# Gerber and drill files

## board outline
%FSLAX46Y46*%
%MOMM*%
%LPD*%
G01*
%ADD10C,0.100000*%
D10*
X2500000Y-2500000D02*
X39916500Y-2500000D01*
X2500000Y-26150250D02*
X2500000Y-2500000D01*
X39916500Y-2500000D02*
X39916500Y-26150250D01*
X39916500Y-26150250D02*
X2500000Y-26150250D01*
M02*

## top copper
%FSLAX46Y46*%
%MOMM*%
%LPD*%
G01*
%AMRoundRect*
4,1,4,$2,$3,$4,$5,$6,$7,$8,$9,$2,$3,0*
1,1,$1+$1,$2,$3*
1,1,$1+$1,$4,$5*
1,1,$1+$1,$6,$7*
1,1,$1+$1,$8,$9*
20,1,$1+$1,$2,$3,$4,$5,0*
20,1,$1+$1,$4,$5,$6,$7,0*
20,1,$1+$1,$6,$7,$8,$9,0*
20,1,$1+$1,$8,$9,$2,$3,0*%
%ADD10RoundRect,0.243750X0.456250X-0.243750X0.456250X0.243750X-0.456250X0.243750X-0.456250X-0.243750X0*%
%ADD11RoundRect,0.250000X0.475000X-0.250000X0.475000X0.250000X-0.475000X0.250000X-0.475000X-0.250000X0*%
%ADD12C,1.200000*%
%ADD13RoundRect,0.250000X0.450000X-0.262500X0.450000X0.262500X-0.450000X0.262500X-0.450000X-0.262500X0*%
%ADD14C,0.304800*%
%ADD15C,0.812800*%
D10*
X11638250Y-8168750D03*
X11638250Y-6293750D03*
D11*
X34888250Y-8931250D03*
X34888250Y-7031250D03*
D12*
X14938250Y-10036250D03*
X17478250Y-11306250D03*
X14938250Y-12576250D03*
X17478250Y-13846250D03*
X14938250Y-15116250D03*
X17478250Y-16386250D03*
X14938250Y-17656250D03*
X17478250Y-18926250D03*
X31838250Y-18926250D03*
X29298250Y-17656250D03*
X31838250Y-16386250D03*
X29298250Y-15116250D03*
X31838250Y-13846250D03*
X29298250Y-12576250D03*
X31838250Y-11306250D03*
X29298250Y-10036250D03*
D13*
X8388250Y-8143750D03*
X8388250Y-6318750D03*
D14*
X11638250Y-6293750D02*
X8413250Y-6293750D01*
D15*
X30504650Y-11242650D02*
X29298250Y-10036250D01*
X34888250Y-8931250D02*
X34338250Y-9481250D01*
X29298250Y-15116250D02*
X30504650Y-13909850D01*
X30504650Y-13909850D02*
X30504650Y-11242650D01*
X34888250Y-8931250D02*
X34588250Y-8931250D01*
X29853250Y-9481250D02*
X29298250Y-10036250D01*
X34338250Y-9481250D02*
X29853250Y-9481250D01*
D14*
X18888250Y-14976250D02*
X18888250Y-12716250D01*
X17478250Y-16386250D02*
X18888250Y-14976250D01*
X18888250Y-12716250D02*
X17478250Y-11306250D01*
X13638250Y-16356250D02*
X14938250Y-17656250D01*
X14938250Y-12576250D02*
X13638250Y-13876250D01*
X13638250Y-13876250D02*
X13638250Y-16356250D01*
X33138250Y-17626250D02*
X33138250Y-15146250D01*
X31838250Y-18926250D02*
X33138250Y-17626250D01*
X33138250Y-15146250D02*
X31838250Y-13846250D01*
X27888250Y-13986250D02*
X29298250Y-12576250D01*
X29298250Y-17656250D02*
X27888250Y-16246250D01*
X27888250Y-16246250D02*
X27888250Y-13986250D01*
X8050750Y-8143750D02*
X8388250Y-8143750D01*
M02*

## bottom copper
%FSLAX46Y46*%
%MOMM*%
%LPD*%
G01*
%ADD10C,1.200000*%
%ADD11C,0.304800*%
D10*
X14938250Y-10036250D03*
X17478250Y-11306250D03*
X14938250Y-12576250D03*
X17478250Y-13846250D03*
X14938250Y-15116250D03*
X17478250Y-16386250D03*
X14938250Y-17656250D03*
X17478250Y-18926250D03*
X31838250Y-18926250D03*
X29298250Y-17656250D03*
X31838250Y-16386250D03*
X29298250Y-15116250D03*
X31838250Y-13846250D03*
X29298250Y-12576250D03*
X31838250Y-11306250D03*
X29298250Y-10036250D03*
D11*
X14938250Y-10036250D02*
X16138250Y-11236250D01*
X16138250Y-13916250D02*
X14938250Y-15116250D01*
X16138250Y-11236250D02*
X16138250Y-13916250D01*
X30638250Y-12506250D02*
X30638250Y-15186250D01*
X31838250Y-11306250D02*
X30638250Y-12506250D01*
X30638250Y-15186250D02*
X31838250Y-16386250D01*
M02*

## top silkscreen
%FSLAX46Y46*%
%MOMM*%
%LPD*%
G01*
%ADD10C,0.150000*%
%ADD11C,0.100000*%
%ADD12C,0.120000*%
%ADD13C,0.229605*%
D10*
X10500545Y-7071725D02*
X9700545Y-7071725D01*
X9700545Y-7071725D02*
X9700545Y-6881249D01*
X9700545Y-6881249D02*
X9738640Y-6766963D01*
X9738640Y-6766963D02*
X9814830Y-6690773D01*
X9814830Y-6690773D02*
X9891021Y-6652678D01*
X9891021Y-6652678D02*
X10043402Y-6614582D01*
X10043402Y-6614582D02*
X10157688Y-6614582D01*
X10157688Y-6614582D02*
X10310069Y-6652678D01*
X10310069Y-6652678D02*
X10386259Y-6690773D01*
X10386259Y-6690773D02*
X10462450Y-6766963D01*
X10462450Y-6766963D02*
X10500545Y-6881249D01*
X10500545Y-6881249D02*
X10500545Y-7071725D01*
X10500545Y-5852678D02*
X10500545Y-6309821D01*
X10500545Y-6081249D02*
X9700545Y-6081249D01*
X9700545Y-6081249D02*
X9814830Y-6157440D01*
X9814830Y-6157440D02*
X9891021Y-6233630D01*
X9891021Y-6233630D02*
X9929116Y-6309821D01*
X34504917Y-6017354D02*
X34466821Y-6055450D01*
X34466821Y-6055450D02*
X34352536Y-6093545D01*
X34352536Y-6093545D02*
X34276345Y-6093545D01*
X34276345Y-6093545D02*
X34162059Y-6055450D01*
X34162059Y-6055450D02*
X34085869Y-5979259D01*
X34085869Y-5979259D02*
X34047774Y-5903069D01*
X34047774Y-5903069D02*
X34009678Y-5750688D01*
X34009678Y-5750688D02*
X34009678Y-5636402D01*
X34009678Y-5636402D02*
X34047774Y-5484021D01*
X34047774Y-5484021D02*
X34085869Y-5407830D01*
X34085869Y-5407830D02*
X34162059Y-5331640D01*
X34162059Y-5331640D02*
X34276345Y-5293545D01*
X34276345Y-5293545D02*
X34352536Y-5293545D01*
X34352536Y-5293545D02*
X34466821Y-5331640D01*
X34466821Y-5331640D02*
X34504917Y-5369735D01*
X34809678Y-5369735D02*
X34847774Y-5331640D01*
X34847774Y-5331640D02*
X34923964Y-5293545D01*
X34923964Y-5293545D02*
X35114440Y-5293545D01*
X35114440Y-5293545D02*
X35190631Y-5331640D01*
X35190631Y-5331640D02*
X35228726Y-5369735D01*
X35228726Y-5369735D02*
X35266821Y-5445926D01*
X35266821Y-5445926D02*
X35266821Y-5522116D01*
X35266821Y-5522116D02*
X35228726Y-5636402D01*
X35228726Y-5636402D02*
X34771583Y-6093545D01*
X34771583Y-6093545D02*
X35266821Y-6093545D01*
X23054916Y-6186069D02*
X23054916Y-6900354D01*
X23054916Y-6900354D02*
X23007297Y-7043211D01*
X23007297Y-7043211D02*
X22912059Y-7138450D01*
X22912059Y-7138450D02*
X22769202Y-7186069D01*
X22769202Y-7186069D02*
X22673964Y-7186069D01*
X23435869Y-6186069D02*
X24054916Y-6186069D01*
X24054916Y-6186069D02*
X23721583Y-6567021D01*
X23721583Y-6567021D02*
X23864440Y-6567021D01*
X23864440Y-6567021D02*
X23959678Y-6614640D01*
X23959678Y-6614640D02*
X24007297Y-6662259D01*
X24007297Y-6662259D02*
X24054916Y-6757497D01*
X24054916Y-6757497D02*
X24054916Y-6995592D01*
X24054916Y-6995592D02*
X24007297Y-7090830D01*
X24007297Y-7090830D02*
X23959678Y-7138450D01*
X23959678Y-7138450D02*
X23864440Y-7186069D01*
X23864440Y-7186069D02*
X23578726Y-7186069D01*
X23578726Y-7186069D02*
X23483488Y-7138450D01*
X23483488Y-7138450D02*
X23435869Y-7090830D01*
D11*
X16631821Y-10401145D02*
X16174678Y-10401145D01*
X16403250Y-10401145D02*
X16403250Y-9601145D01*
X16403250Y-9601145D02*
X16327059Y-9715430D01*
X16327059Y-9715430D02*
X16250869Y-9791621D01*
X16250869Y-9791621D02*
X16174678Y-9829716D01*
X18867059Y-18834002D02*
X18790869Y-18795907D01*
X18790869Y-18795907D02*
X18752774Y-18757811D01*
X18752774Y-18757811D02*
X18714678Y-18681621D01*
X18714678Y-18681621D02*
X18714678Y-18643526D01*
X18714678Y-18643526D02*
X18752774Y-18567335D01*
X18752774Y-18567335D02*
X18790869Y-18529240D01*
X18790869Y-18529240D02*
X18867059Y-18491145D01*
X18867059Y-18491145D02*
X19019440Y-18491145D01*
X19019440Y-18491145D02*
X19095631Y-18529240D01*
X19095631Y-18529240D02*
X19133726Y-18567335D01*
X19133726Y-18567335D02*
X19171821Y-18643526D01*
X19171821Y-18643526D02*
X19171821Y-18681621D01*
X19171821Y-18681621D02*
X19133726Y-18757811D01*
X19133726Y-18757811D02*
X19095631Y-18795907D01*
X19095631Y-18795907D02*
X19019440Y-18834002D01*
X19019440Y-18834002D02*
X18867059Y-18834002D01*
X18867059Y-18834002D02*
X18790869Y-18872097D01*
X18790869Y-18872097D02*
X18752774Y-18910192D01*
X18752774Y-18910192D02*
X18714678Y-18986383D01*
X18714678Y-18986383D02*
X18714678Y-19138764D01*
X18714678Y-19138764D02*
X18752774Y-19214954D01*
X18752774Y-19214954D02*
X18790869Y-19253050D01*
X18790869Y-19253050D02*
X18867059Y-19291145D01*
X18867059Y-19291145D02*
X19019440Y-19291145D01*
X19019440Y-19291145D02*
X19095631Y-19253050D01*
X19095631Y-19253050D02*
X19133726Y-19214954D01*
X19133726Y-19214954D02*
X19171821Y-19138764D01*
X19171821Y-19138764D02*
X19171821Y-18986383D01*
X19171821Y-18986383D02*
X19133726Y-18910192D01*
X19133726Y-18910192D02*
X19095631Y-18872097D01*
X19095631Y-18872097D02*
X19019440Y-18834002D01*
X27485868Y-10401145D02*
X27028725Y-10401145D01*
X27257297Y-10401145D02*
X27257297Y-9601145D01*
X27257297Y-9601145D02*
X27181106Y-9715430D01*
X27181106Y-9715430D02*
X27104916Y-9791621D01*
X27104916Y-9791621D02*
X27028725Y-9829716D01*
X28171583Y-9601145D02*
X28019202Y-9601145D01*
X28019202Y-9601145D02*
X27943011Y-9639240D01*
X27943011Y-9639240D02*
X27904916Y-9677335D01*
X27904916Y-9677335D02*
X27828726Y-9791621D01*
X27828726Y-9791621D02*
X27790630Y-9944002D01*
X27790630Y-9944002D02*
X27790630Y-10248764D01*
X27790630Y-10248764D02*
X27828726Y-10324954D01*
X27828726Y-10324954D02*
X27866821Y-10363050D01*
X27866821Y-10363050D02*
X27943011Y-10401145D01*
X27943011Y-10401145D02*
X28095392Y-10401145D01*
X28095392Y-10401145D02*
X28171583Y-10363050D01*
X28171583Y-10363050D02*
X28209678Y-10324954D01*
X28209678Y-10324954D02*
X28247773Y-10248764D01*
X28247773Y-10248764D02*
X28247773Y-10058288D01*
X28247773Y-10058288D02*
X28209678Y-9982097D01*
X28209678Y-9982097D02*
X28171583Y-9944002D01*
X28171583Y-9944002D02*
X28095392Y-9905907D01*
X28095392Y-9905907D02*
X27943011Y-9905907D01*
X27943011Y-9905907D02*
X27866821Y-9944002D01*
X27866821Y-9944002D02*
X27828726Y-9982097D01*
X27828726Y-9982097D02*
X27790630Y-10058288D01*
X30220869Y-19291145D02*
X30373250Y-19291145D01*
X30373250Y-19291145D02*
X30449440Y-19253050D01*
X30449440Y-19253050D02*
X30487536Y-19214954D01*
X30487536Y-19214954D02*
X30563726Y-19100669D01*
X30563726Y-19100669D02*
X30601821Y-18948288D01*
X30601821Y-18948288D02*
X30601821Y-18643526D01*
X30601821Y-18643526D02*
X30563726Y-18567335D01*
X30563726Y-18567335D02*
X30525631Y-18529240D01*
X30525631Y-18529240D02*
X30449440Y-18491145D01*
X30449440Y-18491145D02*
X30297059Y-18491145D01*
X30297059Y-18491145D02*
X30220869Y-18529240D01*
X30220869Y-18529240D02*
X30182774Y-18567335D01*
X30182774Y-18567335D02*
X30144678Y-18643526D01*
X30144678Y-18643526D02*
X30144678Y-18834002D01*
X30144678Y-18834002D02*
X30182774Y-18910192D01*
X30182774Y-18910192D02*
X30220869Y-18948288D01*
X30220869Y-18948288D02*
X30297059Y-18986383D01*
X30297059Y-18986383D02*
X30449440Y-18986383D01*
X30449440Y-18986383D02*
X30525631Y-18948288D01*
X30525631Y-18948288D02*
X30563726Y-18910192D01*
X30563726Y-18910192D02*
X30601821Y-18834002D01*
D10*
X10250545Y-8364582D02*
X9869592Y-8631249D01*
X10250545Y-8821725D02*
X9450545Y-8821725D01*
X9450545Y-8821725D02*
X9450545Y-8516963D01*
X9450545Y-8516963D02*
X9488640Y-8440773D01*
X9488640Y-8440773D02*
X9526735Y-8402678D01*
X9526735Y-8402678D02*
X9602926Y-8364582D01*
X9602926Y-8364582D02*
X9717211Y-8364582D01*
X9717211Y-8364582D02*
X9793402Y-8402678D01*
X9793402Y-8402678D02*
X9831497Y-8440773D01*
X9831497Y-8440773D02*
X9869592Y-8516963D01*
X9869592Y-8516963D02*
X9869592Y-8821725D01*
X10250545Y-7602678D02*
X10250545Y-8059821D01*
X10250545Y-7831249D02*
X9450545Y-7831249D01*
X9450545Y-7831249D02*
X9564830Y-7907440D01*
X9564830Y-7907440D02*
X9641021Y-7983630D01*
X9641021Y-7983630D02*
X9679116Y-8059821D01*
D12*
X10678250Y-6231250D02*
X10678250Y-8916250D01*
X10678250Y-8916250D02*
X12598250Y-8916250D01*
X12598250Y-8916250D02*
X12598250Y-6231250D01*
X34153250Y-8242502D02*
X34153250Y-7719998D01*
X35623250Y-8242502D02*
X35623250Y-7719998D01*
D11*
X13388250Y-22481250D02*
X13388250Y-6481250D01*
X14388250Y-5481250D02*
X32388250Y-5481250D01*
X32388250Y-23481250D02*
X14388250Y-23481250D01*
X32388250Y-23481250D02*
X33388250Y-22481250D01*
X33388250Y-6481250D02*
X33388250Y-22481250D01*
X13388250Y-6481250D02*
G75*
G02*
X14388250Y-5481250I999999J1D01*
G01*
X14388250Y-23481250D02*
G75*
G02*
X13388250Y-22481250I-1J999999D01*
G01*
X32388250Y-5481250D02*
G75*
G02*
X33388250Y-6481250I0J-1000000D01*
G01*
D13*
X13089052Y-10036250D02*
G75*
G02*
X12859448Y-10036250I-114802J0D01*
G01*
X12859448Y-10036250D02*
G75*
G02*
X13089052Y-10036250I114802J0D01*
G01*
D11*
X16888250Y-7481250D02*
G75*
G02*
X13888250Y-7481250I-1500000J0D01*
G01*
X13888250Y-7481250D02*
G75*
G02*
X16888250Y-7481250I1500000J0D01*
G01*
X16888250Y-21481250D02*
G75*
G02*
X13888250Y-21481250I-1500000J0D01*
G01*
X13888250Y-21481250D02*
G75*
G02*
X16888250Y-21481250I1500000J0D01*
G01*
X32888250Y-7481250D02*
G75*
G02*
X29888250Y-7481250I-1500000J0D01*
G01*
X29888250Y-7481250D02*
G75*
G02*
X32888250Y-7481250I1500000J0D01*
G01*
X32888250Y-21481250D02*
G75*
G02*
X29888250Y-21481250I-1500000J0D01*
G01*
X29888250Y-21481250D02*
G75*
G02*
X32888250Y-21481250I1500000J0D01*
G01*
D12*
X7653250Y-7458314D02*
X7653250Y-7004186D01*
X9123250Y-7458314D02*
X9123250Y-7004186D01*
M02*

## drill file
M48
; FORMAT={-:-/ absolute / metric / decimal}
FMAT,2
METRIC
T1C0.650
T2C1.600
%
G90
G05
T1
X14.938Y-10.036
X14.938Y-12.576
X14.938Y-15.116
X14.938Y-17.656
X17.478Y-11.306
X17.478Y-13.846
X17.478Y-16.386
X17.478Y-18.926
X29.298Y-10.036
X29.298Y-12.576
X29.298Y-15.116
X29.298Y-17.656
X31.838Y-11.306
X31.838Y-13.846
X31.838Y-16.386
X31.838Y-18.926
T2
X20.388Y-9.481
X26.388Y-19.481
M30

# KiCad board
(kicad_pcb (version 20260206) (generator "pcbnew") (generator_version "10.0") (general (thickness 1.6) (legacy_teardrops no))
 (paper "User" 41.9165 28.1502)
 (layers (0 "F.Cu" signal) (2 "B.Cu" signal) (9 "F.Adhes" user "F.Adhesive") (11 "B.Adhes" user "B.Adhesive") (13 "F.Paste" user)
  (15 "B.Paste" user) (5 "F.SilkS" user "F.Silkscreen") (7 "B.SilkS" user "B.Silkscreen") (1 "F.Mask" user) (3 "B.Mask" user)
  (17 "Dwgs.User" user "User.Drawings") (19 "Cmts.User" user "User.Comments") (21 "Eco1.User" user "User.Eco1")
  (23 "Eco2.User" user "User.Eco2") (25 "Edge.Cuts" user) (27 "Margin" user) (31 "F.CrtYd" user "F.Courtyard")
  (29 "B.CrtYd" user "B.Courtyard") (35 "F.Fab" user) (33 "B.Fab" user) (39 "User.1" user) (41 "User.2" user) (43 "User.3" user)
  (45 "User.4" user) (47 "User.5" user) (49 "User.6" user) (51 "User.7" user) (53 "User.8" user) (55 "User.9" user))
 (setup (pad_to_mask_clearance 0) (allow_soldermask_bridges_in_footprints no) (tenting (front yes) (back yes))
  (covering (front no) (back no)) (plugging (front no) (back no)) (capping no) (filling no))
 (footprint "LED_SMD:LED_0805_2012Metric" (layer "F.Cu") (at 11.63825 7.23125 90)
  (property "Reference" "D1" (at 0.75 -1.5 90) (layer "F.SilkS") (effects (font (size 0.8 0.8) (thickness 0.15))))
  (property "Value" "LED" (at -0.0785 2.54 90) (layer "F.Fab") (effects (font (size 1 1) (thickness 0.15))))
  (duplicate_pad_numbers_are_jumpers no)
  (fp_line (start 1 -0.96) (end -1.685 -0.96) (stroke (width 0.12) (type solid)) (layer "F.SilkS"))
  (fp_line (start -1.685 -0.96) (end -1.685 0.96) (stroke (width 0.12) (type solid)) (layer "F.SilkS"))
  (fp_line (start -1.685 0.96) (end 1 0.96) (stroke (width 0.12) (type solid)) (layer "F.SilkS"))
  (pad "1" smd roundrect (at -0.9375 0 90) (size 0.975 1.4) (layers "F.Cu" "F.Mask" "F.Paste") (roundrect_rratio 0.25) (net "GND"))
  (pad "2" smd roundrect (at 0.9375 0 90) (size 0.975 1.4) (layers "F.Cu" "F.Mask" "F.Paste") (roundrect_rratio 0.25) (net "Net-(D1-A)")))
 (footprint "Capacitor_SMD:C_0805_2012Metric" (layer "F.Cu") (at 34.88825 7.98125 90)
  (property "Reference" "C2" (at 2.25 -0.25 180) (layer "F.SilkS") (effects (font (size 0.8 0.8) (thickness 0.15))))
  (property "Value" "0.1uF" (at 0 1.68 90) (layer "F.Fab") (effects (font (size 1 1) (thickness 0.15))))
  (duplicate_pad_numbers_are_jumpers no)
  (fp_line (start -0.261252 -0.735) (end 0.261252 -0.735) (stroke (width 0.12) (type solid)) (layer "F.SilkS"))
  (fp_line (start -0.261252 0.735) (end 0.261252 0.735) (stroke (width 0.12) (type solid)) (layer "F.SilkS"))
  (pad "1" smd roundrect (at -0.95 0 90) (size 1 1.45) (layers "F.Cu" "F.Mask" "F.Paste") (roundrect_rratio 0.25) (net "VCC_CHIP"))
  (pad "2" smd roundrect (at 0.95 0 90) (size 1 1.45) (layers "F.Cu" "F.Mask" "F.Paste") (roundrect_rratio 0.25) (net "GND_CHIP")))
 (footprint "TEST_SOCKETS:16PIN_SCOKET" (layer "F.Cu") (at 23.38825 14.48125)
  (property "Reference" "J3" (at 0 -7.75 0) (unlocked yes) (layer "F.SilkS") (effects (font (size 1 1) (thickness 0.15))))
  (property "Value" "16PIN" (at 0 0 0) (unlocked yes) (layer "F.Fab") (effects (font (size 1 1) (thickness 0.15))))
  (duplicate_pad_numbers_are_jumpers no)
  (fp_line (start -10 8) (end -10 -8) (stroke (width 0.1) (type default)) (layer "F.SilkS"))
  (fp_line (start -9 -9) (end 9 -9) (stroke (width 0.1) (type default)) (layer "F.SilkS"))
  (fp_line (start 9 9) (end -9 9) (stroke (width 0.1) (type default)) (layer "F.SilkS"))
  (fp_line (start 9 9) (end 10 8) (stroke (width 0.1) (type default)) (layer "F.SilkS"))
  (fp_line (start 10 -8) (end 10 8) (stroke (width 0.1) (type default)) (layer "F.SilkS"))
  (fp_arc (start -10 -8) (mid -9.707107 -8.707107) (end -9 -9) (stroke (width 0.1) (type default)) (layer "F.SilkS"))
  (fp_arc (start -9 9) (mid -9.707107 8.707107) (end -10 8) (stroke (width 0.1) (type default)) (layer "F.SilkS"))
  (fp_arc (start 9 -9) (mid 9.707107 -8.707107) (end 10 -8) (stroke (width 0.1) (type default)) (layer "F.SilkS"))
  (fp_circle (center -10.414 -4.445) (end -10.234395 -4.445) (stroke (width 0.1) (type solid)) (fill yes) (layer "F.SilkS"))
  (fp_circle (center -8 -7) (end -6.5 -7) (stroke (width 0.1) (type default)) (fill no) (layer "F.SilkS"))
  (fp_circle (center -8 7) (end -6.5 7) (stroke (width 0.1) (type default)) (fill no) (layer "F.SilkS"))
  (fp_circle (center 8 -7) (end 6.5 -7) (stroke (width 0.1) (type default)) (fill no) (layer "F.SilkS"))
  (fp_circle (center 8 7) (end 6.5 7) (stroke (width 0.1) (type default)) (fill no) (layer "F.SilkS"))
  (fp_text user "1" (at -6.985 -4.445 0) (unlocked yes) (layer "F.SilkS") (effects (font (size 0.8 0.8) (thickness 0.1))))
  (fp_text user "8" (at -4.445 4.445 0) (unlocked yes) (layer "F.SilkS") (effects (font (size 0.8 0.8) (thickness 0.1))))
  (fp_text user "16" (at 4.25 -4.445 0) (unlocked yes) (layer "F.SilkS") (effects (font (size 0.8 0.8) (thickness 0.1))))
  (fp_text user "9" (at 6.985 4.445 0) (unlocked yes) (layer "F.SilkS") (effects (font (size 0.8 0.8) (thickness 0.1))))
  (pad "" np_thru_hole circle (at -3 -5) (size 1.6 1.6) (drill 1.6) (layers "*.Cu" "*.Mask"))
  (pad "" np_thru_hole circle (at 3 5 180) (size 1.6 1.6) (drill 1.6) (layers "*.Cu" "*.Mask"))
  (pad "1" thru_hole circle (at -8.45 -4.445) (size 1.2 1.2) (drill 0.65) (layers "*.Cu" "*.Mask") (remove_unused_layers no) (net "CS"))
  (pad "2" thru_hole circle (at -5.91 -3.175) (size 1.2 1.2) (drill 0.65) (layers "*.Cu" "*.Mask") (remove_unused_layers no) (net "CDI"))
  (pad "3" thru_hole circle (at -8.45 -1.905) (size 1.2 1.2) (drill 0.65) (layers "*.Cu" "*.Mask") (remove_unused_layers no) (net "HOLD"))
  (pad "4" thru_hole circle (at -5.91 -0.635) (size 1.2 1.2) (drill 0.65) (layers "*.Cu" "*.Mask") (remove_unused_layers no)
   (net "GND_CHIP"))
  (pad "5" thru_hole circle (at -8.45 0.635) (size 1.2 1.2) (drill 0.65) (layers "*.Cu" "*.Mask") (remove_unused_layers no) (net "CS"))
  (pad "6" thru_hole circle (at -5.91 1.905) (size 1.2 1.2) (drill 0.65) (layers "*.Cu" "*.Mask") (remove_unused_layers no) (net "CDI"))
  (pad "7" thru_hole circle (at -8.45 3.175) (size 1.2 1.2) (drill 0.65) (layers "*.Cu" "*.Mask") (remove_unused_layers no) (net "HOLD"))
  (pad "8" thru_hole circle (at -5.91 4.445) (size 1.2 1.2) (drill 0.65) (layers "*.Cu" "*.Mask") (remove_unused_layers no) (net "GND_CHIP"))
  (pad "9" thru_hole circle (at 8.45 4.445 180) (size 1.2 1.2) (drill 0.65) (layers "*.Cu" "*.Mask") (remove_unused_layers no) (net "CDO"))
  (pad "10" thru_hole circle (at 5.91 3.175 180) (size 1.2 1.2) (drill 0.65) (layers "*.Cu" "*.Mask") (remove_unused_layers no) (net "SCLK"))
  (pad "11" thru_hole circle (at 8.45 1.905 180) (size 1.2 1.2) (drill 0.65) (layers "*.Cu" "*.Mask") (remove_unused_layers no) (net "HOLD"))
  (pad "12" thru_hole circle (at 5.91 0.635 180) (size 1.2 1.2) (drill 0.65) (layers "*.Cu" "*.Mask") (remove_unused_layers no)
   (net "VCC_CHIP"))
  (pad "13" thru_hole circle (at 8.45 -0.635 180) (size 1.2 1.2) (drill 0.65) (layers "*.Cu" "*.Mask") (remove_unused_layers no) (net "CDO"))
  (pad "14" thru_hole circle (at 5.91 -1.905 180) (size 1.2 1.2) (drill 0.65) (layers "*.Cu" "*.Mask") (remove_unused_layers no)
   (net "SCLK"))
  (pad "15" thru_hole circle (at 8.45 -3.175 180) (size 1.2 1.2) (drill 0.65) (layers "*.Cu" "*.Mask") (remove_unused_layers no)
   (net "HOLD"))
  (pad "16" thru_hole circle (at 5.91 -4.445 180) (size 1.2 1.2) (drill 0.65) (layers "*.Cu" "*.Mask") (remove_unused_layers no)
   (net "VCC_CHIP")))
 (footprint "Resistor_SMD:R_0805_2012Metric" (layer "F.Cu") (at 8.38825 7.23125 90)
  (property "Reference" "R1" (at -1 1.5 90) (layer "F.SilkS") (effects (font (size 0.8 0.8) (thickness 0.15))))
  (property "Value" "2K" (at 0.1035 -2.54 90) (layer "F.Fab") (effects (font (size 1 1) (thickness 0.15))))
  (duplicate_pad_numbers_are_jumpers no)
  (fp_line (start -0.227064 -0.735) (end 0.227064 -0.735) (stroke (width 0.12) (type solid)) (layer "F.SilkS"))
  (fp_line (start -0.227064 0.735) (end 0.227064 0.735) (stroke (width 0.12) (type solid)) (layer "F.SilkS"))
  (pad "1" smd roundrect (at -0.9125 0 90) (size 1.025 1.4) (layers "F.Cu" "F.Mask" "F.Paste") (roundrect_rratio 0.243902439) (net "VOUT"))
  (pad "2" smd roundrect (at 0.9125 0 90) (size 1.025 1.4) (layers "F.Cu" "F.Mask" "F.Paste") (roundrect_rratio 0.243902439)
   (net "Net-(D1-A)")))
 (gr_line (start 2.5 2.5) (end 39.9165 2.5) (stroke (width 0.1) (type default)) (layer "Edge.Cuts"))
 (gr_line (start 2.5 26.15025) (end 2.5 2.5) (stroke (width 0.1) (type default)) (layer "Edge.Cuts"))
 (gr_line (start 39.9165 2.5) (end 39.9165 26.15025) (stroke (width 0.1) (type default)) (layer "Edge.Cuts"))
 (gr_line (start 39.9165 26.15025) (end 2.5 26.15025) (stroke (width 0.1) (type default)) (layer "Edge.Cuts"))
 (segment (start 11.63825 6.29375) (end 8.41325 6.29375) (width 0.3048) (layer "F.Cu") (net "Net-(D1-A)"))
 (segment (start 30.50465 11.24265) (end 29.29825 10.03625) (width 0.8128) (layer "F.Cu") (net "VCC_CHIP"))
 (segment (start 34.88825 8.93125) (end 34.33825 9.48125) (width 0.8128) (layer "F.Cu") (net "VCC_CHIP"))
 (segment (start 29.29825 15.11625) (end 30.50465 13.90985) (width 0.8128) (layer "F.Cu") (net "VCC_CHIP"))
 (segment (start 30.50465 13.90985) (end 30.50465 11.24265) (width 0.8128) (layer "F.Cu") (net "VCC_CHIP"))
 (segment (start 34.88825 8.93125) (end 34.58825 8.93125) (width 0.8128) (layer "F.Cu") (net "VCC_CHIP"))
 (segment (start 29.85325 9.48125) (end 29.29825 10.03625) (width 0.8128) (layer "F.Cu") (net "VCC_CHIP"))
 (segment (start 34.33825 9.48125) (end 29.85325 9.48125) (width 0.8128) (layer "F.Cu") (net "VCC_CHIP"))
 (segment (start 14.93825 10.03625) (end 16.13825 11.23625) (width 0.3048) (layer "B.Cu") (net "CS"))
 (segment (start 16.13825 13.91625) (end 14.93825 15.11625) (width 0.3048) (layer "B.Cu") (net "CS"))
 (segment (start 16.13825 11.23625) (end 16.13825 13.91625) (width 0.3048) (layer "B.Cu") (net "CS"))
 (segment (start 18.88825 14.97625) (end 18.88825 12.71625) (width 0.3048) (layer "F.Cu") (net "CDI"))
 (segment (start 17.47825 16.38625) (end 18.88825 14.97625) (width 0.3048) (layer "F.Cu") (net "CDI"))
 (segment (start 18.88825 12.71625) (end 17.47825 11.30625) (width 0.3048) (layer "F.Cu") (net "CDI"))
 (segment (start 13.63825 16.35625) (end 14.93825 17.65625) (width 0.3048) (layer "F.Cu") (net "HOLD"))
 (segment (start 14.93825 12.57625) (end 13.63825 13.87625) (width 0.3048) (layer "F.Cu") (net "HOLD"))
 (segment (start 13.63825 13.87625) (end 13.63825 16.35625) (width 0.3048) (layer "F.Cu") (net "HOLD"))
 (segment (start 30.63825 12.50625) (end 30.63825 15.18625) (width 0.3048) (layer "B.Cu") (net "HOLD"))
 (segment (start 31.83825 11.30625) (end 30.63825 12.50625) (width 0.3048) (layer "B.Cu") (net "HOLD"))
 (segment (start 30.63825 15.18625) (end 31.83825 16.38625) (width 0.3048) (layer "B.Cu") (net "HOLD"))
 (segment (start 33.13825 17.62625) (end 33.13825 15.14625) (width 0.3048) (layer "F.Cu") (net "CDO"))
 (segment (start 31.83825 18.92625) (end 33.13825 17.62625) (width 0.3048) (layer "F.Cu") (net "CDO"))
 (segment (start 33.13825 15.14625) (end 31.83825 13.84625) (width 0.3048) (layer "F.Cu") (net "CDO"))
 (segment (start 27.88825 13.98625) (end 29.29825 12.57625) (width 0.3048) (layer "F.Cu") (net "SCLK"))
 (segment (start 29.29825 17.65625) (end 27.88825 16.24625) (width 0.3048) (layer "F.Cu") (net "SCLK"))
 (segment (start 27.88825 16.24625) (end 27.88825 13.98625) (width 0.3048) (layer "F.Cu") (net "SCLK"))
 (segment (start 8.05075 8.14375) (end 8.38825 8.14375) (width 0.3048) (layer "F.Cu") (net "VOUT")))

